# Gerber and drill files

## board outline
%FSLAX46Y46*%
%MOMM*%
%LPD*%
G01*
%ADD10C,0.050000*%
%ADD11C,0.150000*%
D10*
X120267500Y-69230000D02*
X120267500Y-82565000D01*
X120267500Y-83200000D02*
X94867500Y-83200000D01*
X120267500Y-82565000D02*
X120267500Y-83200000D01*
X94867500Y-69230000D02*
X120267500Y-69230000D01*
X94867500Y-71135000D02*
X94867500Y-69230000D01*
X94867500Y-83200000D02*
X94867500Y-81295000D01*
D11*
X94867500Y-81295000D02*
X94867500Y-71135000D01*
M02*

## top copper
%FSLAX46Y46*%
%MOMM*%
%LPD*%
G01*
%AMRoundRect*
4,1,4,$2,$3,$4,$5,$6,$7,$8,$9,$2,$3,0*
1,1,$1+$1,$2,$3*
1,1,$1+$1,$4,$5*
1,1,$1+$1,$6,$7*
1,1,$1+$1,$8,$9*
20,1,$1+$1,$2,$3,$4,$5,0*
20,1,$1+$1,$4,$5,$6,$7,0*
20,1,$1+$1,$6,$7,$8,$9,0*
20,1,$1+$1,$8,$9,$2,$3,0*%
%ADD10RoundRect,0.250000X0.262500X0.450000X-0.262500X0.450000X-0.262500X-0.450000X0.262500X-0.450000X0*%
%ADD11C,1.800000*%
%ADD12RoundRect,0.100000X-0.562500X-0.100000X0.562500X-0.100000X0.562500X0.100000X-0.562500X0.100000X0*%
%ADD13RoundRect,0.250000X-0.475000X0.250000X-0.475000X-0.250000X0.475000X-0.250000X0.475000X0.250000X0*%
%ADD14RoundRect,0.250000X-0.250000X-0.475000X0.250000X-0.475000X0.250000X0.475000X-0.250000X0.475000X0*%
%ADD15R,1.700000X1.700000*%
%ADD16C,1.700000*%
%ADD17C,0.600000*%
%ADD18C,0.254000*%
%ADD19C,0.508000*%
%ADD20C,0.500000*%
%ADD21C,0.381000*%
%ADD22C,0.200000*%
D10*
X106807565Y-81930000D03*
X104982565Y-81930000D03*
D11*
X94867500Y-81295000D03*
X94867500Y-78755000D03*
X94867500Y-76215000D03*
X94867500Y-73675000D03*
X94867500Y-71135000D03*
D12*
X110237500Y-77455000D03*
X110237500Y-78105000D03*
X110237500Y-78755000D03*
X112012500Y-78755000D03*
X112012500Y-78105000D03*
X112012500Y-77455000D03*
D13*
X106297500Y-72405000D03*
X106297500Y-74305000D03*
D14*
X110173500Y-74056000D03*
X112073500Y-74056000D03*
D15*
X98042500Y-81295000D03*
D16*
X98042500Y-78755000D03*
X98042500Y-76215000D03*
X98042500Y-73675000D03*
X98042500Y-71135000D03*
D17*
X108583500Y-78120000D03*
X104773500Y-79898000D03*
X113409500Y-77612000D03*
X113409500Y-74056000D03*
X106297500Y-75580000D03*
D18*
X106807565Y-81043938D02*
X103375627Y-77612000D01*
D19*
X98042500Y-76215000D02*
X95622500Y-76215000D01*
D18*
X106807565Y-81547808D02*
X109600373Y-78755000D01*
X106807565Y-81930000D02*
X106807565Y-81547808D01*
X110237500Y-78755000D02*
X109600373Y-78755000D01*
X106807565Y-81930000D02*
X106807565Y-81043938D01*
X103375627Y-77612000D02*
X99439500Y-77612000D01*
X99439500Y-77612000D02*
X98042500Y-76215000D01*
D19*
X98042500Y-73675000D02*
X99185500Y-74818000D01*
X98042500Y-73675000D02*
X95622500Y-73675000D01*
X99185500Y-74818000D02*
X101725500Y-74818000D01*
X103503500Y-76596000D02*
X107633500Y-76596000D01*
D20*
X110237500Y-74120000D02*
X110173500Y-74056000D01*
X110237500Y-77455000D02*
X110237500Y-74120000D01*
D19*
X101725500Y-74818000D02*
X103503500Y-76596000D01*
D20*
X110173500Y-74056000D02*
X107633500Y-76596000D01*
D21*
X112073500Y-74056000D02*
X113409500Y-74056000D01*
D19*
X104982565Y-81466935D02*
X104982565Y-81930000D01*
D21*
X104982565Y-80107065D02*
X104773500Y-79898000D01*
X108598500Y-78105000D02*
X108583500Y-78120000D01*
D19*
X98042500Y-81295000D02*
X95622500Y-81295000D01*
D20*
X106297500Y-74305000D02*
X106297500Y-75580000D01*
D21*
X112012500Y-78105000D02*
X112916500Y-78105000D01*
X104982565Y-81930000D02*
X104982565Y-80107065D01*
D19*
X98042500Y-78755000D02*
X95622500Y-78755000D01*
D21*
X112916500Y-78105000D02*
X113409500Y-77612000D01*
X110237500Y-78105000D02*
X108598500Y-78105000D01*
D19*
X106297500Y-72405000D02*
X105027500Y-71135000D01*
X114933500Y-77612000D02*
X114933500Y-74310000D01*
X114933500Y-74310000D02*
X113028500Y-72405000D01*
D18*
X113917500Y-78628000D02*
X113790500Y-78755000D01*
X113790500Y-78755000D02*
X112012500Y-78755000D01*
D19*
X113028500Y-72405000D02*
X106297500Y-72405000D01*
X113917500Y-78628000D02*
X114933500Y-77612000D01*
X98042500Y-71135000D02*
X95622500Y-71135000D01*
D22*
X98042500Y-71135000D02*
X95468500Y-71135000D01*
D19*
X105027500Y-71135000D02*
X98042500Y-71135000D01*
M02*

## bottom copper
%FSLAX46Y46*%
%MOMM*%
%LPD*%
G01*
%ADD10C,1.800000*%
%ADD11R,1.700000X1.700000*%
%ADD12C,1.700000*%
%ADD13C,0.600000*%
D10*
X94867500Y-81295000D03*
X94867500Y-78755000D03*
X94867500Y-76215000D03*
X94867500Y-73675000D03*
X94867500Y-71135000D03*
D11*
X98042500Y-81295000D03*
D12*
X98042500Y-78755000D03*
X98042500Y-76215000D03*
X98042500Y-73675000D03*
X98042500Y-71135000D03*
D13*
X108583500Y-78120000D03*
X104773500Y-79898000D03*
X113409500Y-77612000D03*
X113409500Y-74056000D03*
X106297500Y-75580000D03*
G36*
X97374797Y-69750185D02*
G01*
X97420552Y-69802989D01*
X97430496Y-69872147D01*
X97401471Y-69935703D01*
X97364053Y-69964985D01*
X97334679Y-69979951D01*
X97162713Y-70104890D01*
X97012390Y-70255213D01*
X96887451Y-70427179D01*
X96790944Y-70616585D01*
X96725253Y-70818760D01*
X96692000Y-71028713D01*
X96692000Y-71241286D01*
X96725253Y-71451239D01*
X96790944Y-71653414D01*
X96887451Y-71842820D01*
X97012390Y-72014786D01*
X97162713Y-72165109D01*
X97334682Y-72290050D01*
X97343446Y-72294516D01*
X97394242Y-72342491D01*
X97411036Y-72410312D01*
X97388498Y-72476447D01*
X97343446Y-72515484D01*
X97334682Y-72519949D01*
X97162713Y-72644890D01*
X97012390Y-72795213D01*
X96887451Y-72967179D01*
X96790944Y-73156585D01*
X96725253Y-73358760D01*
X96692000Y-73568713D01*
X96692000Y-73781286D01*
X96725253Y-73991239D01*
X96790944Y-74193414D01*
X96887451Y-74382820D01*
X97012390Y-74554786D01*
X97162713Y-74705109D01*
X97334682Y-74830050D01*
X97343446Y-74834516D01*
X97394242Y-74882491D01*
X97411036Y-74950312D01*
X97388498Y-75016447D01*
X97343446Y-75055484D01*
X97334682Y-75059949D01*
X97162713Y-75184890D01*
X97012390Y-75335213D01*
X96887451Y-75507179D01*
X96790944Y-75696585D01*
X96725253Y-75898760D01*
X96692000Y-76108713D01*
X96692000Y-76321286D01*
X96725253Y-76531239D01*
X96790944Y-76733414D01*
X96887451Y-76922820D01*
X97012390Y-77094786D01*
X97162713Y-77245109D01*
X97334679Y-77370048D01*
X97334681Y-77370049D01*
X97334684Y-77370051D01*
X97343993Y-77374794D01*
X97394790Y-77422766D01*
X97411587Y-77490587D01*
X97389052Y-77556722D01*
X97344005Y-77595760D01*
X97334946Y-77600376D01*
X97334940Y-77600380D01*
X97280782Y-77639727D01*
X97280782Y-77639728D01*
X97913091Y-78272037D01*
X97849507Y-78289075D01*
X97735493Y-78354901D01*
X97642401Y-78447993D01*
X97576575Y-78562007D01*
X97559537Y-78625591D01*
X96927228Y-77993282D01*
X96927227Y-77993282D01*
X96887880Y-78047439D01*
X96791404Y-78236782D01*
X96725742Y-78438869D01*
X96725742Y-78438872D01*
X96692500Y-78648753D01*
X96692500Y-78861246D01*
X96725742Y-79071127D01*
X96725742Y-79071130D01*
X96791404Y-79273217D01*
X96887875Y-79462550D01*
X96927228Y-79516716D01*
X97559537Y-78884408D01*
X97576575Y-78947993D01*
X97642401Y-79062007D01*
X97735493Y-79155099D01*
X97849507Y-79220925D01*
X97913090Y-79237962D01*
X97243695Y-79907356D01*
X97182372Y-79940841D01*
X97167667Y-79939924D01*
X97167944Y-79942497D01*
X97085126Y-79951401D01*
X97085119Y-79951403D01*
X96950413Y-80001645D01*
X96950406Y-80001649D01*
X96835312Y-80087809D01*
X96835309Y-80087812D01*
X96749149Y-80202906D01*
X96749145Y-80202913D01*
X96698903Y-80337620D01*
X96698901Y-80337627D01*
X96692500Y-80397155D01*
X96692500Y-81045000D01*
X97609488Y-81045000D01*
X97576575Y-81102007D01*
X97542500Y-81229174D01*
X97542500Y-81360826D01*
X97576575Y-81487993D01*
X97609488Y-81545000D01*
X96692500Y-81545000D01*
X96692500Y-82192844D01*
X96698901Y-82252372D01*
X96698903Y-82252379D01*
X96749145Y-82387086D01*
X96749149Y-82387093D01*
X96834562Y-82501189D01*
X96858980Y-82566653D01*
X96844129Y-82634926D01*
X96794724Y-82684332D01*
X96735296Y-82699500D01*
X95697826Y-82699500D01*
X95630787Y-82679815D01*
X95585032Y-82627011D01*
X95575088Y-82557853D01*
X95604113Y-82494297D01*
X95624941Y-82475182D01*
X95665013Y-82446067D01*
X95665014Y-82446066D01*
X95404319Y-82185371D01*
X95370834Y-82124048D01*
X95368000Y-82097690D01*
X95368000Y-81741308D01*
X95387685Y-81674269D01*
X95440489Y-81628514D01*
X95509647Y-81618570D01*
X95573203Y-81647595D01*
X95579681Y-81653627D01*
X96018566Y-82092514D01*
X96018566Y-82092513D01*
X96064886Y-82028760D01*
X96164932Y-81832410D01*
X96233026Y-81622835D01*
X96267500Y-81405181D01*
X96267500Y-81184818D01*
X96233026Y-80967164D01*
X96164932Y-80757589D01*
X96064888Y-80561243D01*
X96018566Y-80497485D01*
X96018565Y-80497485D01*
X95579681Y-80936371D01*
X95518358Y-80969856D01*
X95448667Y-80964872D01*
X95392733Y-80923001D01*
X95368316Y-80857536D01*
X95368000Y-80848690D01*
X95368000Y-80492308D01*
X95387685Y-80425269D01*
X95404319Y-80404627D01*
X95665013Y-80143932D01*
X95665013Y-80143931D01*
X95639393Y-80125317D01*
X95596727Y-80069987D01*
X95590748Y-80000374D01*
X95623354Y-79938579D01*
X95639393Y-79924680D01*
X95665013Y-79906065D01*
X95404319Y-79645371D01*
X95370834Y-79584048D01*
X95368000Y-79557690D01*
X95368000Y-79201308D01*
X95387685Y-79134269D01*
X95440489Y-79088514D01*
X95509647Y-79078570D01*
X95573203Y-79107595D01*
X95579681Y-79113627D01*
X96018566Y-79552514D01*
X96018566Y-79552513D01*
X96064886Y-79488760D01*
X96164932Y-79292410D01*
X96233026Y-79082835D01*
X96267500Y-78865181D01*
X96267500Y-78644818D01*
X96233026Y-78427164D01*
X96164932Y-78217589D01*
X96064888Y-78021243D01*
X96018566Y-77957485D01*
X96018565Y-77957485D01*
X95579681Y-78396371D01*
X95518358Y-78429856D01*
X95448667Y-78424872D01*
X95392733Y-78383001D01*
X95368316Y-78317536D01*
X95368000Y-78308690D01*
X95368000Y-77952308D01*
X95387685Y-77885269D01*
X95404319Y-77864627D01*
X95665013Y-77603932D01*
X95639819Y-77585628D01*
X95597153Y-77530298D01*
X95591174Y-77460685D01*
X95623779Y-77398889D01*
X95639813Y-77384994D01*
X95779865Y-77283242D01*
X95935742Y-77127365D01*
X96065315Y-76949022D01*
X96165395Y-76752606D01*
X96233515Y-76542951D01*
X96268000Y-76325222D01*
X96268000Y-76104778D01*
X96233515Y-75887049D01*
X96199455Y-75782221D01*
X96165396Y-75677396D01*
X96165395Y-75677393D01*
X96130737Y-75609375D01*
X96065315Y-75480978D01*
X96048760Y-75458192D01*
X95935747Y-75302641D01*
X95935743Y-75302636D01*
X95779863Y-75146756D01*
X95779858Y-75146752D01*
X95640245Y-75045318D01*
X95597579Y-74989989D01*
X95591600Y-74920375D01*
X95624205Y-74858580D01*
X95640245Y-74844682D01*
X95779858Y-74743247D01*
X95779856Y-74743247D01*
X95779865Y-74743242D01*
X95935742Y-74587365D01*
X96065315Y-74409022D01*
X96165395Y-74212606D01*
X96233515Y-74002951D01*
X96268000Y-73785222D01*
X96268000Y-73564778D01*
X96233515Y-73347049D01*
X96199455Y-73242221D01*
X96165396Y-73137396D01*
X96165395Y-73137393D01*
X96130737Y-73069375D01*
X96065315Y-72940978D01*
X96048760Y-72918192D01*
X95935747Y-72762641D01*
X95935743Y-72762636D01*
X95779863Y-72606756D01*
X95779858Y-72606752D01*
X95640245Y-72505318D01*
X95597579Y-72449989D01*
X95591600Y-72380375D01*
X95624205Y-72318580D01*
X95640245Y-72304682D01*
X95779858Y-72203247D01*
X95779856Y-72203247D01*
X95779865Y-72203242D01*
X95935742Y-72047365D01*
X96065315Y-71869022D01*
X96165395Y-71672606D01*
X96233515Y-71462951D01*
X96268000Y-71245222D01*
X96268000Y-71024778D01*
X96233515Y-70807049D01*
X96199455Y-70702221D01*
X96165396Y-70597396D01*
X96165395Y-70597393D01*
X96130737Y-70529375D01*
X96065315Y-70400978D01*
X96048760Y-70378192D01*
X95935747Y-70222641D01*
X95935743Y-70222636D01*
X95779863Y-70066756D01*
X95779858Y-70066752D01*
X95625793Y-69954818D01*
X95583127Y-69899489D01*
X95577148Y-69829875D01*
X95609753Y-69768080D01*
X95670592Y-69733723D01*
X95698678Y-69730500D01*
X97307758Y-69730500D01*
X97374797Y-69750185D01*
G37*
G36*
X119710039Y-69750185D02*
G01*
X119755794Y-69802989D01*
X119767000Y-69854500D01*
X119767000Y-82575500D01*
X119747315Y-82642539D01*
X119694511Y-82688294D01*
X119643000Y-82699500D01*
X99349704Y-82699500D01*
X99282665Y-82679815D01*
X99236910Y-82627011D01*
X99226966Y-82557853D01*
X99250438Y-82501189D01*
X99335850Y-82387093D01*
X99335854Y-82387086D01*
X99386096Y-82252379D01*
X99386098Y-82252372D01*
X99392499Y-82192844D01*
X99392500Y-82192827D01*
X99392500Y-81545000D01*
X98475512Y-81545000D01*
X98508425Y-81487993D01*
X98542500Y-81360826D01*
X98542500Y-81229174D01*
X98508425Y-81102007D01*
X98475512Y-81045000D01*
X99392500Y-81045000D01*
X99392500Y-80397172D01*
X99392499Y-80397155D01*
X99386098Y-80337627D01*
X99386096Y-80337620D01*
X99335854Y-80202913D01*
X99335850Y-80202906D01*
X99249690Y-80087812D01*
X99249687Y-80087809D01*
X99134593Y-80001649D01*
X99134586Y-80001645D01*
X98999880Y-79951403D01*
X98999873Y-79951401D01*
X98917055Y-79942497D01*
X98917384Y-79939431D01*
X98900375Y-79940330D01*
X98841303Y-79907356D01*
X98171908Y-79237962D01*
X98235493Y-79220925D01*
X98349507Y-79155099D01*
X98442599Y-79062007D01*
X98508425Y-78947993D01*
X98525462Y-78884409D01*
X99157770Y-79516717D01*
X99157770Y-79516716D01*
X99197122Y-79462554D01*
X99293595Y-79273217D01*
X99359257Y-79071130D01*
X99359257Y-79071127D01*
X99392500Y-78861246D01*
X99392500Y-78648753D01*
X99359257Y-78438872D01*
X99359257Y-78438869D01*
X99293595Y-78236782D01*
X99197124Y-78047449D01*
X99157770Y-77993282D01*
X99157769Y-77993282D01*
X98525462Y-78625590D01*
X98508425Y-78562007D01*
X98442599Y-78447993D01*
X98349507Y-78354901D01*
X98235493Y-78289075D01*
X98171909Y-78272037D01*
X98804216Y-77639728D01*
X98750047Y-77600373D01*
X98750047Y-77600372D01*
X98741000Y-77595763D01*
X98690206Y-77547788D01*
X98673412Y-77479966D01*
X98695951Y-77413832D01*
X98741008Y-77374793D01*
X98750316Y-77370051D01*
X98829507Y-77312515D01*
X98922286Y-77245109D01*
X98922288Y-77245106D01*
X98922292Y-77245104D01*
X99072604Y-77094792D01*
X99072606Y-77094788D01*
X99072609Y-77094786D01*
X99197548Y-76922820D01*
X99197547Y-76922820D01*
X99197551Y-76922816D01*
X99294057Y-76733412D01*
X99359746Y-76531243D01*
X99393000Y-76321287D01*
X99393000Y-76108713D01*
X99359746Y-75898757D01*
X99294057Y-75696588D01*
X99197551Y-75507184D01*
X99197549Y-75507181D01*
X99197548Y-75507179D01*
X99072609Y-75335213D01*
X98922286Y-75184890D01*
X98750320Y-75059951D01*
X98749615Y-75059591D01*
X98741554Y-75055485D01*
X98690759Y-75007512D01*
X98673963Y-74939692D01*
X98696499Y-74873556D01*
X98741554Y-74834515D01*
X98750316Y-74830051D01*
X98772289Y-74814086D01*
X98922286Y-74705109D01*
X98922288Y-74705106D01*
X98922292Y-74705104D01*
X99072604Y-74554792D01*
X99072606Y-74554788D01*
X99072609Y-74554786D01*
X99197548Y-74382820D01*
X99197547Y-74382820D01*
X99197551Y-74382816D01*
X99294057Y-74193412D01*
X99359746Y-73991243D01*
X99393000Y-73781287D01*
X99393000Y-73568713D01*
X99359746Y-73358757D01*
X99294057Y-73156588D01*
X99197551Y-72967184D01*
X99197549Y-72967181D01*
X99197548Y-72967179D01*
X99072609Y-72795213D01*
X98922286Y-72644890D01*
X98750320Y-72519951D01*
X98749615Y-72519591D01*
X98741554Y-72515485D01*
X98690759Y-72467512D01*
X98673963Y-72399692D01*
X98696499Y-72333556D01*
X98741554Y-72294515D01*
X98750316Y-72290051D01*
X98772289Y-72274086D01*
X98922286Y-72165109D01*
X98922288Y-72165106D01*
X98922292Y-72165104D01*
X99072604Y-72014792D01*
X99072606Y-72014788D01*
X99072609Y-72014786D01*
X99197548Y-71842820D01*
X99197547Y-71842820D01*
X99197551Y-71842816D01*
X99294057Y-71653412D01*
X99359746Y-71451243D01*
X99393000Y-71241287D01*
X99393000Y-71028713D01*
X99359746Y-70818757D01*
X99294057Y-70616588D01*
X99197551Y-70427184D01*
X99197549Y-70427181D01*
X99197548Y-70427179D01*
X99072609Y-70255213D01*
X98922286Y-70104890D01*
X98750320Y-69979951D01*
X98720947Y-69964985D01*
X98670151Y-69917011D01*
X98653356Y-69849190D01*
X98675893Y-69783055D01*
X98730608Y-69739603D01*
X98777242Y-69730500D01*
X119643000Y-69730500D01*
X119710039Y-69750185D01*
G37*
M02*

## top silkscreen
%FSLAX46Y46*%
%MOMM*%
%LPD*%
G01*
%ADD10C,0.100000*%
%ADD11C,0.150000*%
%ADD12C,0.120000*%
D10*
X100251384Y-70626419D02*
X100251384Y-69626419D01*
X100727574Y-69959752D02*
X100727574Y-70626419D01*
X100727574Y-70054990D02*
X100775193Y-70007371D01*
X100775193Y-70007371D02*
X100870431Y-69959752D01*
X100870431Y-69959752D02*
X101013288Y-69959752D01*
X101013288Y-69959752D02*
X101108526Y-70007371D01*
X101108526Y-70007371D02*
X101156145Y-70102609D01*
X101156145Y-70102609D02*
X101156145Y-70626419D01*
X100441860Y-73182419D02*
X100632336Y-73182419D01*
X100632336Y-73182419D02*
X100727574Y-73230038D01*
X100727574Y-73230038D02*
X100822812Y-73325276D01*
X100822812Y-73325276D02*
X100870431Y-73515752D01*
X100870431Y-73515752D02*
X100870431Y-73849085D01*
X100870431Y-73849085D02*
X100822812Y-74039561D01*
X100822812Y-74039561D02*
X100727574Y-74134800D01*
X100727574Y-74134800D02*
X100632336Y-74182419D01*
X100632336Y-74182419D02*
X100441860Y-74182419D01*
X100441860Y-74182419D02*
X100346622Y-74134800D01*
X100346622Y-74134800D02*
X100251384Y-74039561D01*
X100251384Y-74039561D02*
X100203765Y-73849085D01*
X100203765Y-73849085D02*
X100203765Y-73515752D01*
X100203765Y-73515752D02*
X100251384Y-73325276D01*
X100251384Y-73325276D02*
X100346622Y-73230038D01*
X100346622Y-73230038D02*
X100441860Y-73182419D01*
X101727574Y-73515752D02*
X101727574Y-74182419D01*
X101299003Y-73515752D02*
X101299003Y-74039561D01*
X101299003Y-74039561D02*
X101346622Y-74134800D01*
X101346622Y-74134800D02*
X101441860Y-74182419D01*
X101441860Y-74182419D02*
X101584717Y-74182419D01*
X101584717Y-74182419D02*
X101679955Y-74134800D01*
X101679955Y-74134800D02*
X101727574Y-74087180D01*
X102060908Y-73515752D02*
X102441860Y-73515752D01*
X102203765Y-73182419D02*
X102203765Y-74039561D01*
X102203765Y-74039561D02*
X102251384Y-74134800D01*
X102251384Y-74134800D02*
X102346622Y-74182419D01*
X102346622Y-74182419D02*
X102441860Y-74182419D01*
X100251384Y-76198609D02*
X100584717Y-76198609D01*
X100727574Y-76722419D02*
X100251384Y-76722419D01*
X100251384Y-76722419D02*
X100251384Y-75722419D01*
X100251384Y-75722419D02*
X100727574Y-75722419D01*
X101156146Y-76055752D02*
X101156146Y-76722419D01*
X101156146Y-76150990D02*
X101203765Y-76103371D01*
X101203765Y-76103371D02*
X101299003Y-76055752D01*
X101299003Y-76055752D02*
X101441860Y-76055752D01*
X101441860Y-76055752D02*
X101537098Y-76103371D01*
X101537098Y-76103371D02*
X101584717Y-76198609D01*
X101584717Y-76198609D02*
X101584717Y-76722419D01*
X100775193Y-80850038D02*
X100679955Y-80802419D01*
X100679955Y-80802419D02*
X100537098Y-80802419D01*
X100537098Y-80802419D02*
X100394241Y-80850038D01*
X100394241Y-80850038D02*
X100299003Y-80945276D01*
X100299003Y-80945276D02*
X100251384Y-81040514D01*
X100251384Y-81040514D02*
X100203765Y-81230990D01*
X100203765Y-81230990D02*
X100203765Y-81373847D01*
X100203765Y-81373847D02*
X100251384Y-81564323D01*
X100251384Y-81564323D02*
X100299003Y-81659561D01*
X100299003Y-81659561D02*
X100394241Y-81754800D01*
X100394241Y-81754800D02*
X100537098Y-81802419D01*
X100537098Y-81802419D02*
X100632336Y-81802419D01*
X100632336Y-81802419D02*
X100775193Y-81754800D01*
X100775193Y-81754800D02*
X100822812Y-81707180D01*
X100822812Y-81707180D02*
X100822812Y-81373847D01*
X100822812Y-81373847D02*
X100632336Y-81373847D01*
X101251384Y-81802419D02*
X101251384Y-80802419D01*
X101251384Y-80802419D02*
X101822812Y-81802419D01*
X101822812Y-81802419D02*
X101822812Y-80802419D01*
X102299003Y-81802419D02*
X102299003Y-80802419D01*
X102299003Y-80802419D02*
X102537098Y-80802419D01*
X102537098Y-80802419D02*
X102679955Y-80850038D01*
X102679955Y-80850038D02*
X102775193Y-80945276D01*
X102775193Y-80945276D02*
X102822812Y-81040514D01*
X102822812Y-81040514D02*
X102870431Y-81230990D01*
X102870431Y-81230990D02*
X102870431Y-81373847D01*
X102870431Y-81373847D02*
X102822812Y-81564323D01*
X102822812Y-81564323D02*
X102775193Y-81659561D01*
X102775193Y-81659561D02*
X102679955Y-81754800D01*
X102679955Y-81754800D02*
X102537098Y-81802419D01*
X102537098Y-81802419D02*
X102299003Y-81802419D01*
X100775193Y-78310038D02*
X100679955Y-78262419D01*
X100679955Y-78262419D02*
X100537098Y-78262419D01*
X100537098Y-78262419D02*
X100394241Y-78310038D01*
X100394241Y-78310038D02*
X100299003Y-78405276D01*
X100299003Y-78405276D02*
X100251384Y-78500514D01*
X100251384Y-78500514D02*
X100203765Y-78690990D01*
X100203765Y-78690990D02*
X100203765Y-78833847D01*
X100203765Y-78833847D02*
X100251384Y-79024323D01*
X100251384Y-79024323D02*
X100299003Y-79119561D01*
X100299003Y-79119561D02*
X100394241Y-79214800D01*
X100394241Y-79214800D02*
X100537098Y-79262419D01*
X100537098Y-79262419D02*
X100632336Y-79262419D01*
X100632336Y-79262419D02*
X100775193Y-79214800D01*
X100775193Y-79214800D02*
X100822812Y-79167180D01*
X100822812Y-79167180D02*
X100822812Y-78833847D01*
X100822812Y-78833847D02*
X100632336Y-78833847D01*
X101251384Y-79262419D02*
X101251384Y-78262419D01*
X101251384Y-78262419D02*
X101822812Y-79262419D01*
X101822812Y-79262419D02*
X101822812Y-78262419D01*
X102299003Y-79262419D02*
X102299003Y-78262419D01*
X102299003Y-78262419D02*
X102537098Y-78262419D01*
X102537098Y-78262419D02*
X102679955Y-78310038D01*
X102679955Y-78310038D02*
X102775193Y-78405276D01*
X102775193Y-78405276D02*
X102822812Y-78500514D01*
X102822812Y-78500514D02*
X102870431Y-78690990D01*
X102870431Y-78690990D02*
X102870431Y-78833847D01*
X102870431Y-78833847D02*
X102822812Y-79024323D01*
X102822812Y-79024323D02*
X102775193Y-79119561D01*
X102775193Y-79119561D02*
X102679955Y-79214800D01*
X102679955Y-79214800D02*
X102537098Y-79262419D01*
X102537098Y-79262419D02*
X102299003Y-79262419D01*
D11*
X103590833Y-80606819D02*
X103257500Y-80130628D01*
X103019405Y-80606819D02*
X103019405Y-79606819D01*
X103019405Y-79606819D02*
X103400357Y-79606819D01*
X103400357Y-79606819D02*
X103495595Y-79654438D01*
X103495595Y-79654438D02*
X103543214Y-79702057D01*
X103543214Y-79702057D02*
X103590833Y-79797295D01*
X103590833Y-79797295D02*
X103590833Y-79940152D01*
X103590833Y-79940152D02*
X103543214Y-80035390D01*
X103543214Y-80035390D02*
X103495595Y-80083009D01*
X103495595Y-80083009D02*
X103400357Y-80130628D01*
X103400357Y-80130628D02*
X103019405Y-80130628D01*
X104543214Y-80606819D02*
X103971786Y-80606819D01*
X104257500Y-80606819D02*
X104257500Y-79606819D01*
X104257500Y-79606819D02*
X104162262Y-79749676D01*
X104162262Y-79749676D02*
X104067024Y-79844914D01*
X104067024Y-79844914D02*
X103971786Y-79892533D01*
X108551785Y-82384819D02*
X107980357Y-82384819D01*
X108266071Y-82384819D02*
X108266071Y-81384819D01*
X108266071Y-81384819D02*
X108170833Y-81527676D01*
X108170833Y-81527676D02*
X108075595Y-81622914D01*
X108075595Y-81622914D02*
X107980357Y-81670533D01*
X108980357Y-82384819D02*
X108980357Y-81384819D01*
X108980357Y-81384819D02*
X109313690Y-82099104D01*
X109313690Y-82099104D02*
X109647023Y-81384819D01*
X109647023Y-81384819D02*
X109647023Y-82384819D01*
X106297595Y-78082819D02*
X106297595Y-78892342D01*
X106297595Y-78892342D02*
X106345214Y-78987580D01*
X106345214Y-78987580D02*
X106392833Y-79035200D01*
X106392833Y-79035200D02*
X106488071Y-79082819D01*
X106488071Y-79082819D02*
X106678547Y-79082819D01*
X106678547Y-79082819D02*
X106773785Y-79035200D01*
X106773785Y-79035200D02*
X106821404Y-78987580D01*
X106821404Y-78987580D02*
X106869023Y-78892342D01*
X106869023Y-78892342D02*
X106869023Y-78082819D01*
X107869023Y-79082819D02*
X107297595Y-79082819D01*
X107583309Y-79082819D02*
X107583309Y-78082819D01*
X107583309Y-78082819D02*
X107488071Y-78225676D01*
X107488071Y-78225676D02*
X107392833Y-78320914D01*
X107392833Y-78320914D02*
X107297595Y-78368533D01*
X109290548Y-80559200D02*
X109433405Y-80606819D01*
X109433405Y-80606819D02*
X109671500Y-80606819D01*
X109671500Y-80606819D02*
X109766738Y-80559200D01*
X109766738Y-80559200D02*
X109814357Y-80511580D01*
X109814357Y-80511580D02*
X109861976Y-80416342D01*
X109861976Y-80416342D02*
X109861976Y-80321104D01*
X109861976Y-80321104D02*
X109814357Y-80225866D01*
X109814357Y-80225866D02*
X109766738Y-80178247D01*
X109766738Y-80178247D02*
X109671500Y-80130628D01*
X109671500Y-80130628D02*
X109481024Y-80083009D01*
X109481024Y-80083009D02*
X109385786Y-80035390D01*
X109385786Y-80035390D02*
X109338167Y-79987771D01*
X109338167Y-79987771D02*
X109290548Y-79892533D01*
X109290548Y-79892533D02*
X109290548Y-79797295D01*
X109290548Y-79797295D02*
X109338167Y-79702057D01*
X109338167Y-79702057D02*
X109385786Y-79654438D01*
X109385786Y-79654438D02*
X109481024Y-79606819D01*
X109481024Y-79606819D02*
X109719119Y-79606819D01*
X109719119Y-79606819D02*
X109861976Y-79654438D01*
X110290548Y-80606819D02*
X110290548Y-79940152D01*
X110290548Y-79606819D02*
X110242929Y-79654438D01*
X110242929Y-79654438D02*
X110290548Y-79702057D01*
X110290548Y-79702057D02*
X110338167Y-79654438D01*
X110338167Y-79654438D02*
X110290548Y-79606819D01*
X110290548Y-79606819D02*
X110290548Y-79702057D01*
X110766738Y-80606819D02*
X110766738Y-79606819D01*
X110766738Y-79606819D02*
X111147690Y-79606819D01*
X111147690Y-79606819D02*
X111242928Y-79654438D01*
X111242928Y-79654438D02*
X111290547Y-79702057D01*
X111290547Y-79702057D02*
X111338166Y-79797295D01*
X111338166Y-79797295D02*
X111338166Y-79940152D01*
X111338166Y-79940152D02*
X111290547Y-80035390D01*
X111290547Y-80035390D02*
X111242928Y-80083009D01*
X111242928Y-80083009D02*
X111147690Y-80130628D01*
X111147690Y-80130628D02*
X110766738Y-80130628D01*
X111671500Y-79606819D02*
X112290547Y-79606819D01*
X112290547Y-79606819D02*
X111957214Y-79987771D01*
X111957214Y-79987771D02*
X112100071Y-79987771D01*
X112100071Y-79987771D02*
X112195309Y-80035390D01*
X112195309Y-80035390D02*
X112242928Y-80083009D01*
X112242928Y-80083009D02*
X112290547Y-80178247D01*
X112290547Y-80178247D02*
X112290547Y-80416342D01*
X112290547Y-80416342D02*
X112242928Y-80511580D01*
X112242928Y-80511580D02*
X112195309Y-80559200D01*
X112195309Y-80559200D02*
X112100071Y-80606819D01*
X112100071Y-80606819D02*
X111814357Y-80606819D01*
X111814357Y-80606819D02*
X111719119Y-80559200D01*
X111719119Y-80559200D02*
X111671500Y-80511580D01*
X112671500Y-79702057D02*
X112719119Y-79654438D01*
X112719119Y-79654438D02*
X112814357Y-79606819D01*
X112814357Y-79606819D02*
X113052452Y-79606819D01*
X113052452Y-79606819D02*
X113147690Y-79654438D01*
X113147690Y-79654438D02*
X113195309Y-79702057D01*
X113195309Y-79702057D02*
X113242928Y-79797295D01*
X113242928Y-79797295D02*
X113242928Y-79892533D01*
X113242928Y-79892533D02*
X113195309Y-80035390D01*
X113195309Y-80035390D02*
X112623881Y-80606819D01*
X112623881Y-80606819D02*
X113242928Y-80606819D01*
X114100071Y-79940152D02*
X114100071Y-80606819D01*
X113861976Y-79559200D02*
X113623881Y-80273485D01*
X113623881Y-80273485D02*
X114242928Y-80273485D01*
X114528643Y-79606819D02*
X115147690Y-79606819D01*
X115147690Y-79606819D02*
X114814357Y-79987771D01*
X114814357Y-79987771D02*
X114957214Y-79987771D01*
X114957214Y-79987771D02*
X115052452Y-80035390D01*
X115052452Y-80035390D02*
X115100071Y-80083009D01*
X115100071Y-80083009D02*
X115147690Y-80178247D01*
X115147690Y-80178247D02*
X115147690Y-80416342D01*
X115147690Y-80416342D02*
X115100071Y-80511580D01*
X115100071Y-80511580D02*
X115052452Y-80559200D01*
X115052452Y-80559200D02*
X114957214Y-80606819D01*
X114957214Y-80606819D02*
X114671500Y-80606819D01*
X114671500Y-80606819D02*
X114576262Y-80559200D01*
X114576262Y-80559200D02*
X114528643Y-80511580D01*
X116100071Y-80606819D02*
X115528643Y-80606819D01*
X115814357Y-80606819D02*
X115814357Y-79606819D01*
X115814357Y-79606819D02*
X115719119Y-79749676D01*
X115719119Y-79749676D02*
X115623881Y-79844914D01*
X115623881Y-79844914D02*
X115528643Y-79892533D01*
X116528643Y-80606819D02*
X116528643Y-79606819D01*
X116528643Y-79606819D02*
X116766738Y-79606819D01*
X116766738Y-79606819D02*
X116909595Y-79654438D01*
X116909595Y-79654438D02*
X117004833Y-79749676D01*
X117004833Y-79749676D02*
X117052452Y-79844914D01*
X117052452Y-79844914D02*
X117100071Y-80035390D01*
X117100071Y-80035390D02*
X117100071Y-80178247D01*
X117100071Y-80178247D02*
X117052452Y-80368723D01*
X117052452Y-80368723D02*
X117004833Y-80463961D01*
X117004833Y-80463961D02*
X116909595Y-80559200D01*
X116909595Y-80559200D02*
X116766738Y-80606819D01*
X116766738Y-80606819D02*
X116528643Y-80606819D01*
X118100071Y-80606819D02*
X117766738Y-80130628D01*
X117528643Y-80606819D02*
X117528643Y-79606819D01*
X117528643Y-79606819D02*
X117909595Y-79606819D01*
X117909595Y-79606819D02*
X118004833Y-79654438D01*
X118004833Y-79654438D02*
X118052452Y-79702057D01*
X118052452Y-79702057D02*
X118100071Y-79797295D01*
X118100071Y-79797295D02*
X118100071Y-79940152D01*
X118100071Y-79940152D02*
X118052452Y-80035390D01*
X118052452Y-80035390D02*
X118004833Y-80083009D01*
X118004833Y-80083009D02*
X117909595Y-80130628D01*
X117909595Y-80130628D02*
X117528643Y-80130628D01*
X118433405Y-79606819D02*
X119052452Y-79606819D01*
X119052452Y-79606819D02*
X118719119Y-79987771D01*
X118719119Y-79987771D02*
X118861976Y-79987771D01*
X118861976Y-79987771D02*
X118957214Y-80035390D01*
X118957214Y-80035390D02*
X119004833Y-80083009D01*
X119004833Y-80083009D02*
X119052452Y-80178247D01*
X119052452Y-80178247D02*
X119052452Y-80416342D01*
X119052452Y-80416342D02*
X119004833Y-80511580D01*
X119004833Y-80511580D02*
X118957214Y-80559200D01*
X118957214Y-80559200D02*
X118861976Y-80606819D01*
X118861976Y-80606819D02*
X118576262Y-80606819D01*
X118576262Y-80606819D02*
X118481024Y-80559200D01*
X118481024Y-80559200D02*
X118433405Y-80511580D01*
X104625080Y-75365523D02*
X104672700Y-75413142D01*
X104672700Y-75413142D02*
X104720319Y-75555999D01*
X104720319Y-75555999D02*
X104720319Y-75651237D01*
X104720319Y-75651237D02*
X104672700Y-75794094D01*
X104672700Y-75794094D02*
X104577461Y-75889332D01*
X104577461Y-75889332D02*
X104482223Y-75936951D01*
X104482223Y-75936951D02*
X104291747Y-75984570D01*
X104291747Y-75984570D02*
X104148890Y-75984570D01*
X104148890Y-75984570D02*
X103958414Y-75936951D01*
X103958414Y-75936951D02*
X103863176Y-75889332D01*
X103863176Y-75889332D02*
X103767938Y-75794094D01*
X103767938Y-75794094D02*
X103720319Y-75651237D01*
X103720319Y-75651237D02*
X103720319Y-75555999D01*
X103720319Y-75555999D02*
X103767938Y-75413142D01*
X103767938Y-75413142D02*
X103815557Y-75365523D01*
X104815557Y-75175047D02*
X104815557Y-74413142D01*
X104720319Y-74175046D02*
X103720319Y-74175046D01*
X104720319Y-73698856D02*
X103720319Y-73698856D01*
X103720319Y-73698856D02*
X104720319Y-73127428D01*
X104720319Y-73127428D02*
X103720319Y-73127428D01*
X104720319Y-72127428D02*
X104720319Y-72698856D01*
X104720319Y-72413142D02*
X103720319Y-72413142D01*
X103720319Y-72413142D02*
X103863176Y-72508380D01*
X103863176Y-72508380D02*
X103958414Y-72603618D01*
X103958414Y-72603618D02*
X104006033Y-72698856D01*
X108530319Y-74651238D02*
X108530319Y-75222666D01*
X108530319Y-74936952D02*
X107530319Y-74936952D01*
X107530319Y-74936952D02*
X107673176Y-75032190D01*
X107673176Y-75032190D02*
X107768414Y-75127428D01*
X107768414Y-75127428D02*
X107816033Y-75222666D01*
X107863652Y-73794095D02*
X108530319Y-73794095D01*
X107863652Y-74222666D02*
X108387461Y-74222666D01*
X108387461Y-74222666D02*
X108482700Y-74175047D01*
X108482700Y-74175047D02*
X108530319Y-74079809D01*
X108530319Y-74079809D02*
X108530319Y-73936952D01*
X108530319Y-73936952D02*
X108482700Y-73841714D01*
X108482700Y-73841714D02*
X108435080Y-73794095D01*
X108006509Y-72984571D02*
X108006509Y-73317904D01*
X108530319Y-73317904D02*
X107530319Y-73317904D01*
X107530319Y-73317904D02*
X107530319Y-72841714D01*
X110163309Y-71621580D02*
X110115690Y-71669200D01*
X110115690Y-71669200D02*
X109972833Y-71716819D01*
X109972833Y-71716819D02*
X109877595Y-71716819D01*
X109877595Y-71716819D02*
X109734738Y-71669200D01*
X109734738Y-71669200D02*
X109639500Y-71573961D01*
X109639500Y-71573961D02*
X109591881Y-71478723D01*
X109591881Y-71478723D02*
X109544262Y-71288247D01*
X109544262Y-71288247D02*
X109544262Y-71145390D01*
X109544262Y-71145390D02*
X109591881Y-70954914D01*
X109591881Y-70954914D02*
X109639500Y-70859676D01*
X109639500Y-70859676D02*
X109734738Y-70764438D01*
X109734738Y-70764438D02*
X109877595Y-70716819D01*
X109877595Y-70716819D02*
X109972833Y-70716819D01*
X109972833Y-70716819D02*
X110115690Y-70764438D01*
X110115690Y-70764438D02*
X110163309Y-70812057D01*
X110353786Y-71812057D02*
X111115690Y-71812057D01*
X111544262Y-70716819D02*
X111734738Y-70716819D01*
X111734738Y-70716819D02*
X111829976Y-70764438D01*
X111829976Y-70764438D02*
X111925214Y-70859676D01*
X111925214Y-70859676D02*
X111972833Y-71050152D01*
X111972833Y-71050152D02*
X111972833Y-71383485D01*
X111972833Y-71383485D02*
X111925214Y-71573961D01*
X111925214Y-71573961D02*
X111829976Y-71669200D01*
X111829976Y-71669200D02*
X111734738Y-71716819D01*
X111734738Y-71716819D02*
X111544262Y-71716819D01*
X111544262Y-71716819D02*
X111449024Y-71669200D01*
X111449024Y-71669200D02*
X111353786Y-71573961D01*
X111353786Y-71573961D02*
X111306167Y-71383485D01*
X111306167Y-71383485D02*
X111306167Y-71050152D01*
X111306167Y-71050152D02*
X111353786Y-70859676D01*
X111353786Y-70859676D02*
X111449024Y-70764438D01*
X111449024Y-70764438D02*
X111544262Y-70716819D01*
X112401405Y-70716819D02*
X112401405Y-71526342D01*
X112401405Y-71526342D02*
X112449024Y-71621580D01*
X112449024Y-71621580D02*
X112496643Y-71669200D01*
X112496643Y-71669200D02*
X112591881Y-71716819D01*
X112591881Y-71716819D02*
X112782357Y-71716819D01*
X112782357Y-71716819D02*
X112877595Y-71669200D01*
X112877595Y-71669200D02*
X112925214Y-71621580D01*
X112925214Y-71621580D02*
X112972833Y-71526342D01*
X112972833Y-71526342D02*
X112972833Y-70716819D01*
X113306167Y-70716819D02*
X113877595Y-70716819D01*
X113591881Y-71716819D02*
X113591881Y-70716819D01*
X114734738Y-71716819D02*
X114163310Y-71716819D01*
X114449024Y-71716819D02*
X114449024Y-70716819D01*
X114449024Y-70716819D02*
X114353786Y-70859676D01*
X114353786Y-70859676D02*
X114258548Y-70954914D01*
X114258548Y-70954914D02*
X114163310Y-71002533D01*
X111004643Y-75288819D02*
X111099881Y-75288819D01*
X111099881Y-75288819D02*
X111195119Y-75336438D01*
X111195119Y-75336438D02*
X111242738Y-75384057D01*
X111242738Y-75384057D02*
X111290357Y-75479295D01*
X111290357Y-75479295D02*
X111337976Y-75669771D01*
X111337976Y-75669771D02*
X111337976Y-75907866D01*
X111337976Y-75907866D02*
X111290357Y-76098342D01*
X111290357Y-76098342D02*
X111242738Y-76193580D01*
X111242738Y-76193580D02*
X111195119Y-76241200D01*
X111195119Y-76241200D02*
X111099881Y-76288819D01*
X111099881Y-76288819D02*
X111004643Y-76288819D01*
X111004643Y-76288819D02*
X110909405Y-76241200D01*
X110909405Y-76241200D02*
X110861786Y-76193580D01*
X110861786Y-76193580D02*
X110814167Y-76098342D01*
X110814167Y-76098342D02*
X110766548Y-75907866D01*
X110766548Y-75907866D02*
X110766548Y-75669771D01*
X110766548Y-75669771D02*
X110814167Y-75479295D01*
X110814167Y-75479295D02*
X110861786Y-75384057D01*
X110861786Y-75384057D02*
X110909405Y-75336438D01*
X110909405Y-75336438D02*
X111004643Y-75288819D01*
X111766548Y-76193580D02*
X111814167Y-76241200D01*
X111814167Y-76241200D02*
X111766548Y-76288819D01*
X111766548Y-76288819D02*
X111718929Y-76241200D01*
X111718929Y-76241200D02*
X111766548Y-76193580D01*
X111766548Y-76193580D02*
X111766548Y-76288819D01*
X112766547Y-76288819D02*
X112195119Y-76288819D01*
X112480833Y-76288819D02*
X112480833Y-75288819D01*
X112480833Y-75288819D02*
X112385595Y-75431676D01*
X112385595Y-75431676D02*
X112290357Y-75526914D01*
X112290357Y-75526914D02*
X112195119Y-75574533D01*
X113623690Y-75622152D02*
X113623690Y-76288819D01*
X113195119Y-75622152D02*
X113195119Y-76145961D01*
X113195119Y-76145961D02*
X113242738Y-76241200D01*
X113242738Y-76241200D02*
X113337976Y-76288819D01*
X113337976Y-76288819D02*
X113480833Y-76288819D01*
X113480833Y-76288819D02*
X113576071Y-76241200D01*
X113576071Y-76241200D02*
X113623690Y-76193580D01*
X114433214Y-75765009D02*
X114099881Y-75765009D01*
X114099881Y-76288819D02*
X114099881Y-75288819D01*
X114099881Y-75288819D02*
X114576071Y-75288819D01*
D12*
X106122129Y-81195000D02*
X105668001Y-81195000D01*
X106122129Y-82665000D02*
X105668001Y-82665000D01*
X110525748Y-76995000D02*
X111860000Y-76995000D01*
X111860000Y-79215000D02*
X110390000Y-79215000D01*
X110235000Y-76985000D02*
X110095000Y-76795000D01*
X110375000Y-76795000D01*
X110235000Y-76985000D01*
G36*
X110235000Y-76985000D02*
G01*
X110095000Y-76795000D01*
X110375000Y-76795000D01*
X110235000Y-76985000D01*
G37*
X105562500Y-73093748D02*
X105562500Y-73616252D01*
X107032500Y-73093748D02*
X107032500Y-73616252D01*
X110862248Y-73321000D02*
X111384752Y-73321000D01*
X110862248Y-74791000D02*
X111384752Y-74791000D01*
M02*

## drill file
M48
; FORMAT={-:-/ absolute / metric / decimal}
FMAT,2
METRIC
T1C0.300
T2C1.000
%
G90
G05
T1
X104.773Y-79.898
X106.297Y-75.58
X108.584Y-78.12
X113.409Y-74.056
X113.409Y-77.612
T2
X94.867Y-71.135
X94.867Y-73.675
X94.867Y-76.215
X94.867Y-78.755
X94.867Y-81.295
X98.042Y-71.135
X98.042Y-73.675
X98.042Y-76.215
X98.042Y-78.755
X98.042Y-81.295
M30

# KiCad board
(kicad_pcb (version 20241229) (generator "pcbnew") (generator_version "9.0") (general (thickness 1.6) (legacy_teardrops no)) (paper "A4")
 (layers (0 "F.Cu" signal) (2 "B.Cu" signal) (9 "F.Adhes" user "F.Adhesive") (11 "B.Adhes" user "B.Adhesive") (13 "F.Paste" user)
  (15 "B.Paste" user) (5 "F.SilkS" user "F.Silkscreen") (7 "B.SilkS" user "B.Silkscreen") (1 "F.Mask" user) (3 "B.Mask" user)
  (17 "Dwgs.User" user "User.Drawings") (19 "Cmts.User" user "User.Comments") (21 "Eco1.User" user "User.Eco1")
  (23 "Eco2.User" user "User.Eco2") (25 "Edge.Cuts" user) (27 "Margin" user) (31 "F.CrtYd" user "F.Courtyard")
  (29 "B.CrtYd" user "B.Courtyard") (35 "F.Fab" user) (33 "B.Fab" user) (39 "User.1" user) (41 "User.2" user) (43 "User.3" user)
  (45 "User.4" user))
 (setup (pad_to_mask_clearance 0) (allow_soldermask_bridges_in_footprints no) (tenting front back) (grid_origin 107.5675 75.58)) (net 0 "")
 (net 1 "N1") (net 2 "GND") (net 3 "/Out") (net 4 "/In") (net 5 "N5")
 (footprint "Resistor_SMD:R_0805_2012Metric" (layer "F.Cu") (at 105.895065 81.93 180)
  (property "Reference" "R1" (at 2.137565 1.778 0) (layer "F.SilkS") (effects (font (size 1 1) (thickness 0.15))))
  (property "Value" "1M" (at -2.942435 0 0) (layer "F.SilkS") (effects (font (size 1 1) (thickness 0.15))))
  (fp_line (start -0.227064 0.735) (end 0.227064 0.735) (stroke (width 0.12) (type solid)) (layer "F.SilkS"))
  (fp_line (start -0.227064 -0.735) (end 0.227064 -0.735) (stroke (width 0.12) (type solid)) (layer "F.SilkS"))
  (pad "1" smd roundrect (at -0.9125 0 180) (size 1.025 1.4) (layers "F.Cu" "F.Mask" "F.Paste") (roundrect_rratio 0.243902) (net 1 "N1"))
  (pad "2" smd roundrect (at 0.9125 0 180) (size 1.025 1.4) (layers "F.Cu" "F.Mask" "F.Paste") (roundrect_rratio 0.243902) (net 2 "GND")))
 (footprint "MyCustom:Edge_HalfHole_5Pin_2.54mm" (layer "F.Cu") (at 94.8675 81.295 90)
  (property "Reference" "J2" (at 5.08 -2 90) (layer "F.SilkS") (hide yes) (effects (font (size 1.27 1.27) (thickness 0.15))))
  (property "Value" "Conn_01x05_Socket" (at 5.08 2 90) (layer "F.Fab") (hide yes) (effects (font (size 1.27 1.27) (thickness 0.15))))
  (fp_line (start 0 0) (end 10.16 0) (stroke (width 0.15) (type solid)) (layer "Edge.Cuts"))
  (pad "1" thru_hole circle (at 0 0 90) (size 1.8 1.8) (drill 1) (layers "*.Cu" "*.Mask") (remove_unused_layers no) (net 2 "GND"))
  (pad "2" thru_hole circle (at 2.54 0 90) (size 1.8 1.8) (drill 1) (layers "*.Cu" "*.Mask") (remove_unused_layers no) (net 2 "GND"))
  (pad "3" thru_hole circle (at 5.08 0 90) (size 1.8 1.8) (drill 1) (layers "*.Cu" "*.Mask") (remove_unused_layers no) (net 1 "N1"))
  (pad "4" thru_hole circle (at 7.62 0 90) (size 1.8 1.8) (drill 1) (layers "*.Cu" "*.Mask") (remove_unused_layers no) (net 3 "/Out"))
  (pad "5" thru_hole circle (at 10.16 0 90) (size 1.8 1.8) (drill 1) (layers "*.Cu" "*.Mask") (remove_unused_layers no) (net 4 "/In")))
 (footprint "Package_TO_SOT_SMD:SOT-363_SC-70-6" (layer "F.Cu") (at 111.125 78.105)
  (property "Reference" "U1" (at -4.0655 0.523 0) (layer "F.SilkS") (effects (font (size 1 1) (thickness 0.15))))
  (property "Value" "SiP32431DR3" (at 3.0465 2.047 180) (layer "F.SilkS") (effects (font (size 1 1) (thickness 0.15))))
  (fp_line (start -0.599252 -1.11) (end 0.735 -1.11) (stroke (width 0.12) (type solid)) (layer "F.SilkS"))
  (fp_line (start 0.735 1.11) (end -0.735 1.11) (stroke (width 0.12) (type solid)) (layer "F.SilkS"))
  (fp_poly (pts (xy -0.89 -1.12) (xy -1.03 -1.31) (xy -0.75 -1.31)) (stroke (width 0.12) (type solid)) (fill yes) (layer "F.SilkS"))
  (pad "1" smd roundrect (at -0.8875 -0.65) (size 1.325 0.4) (layers "F.Cu" "F.Mask" "F.Paste") (roundrect_rratio 0.25) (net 3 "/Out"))
  (pad "2" smd roundrect (at -0.8875 0) (size 1.325 0.4) (layers "F.Cu" "F.Mask" "F.Paste") (roundrect_rratio 0.25) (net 2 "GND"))
  (pad "3" smd roundrect (at -0.8875 0.65) (size 1.325 0.4) (layers "F.Cu" "F.Mask" "F.Paste") (roundrect_rratio 0.25) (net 1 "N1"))
  (pad "4" smd roundrect (at 0.8875 0.65) (size 1.325 0.4) (layers "F.Cu" "F.Mask" "F.Paste") (roundrect_rratio 0.25) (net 4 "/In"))
  (pad "5" smd roundrect (at 0.8875 0) (size 1.325 0.4) (layers "F.Cu" "F.Mask" "F.Paste") (roundrect_rratio 0.25) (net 2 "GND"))
  (pad "6" smd roundrect (at 0.8875 -0.65) (size 1.325 0.4) (layers "F.Cu" "F.Mask" "F.Paste") (roundrect_rratio 0.25) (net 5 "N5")))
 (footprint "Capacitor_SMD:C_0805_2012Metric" (layer "F.Cu") (at 106.2975 73.355 -90)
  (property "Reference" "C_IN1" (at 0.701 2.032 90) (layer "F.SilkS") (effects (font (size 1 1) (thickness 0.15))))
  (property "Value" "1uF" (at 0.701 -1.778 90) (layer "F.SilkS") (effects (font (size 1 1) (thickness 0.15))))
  (fp_line (start -0.261252 0.735) (end 0.261252 0.735) (stroke (width 0.12) (type solid)) (layer "F.SilkS"))
  (fp_line (start -0.261252 -0.735) (end 0.261252 -0.735) (stroke (width 0.12) (type solid)) (layer "F.SilkS"))
  (pad "1" smd roundrect (at -0.95 0 270) (size 1 1.45) (layers "F.Cu" "F.Mask" "F.Paste") (roundrect_rratio 0.25) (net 4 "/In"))
  (pad "2" smd roundrect (at 0.95 0 270) (size 1 1.45) (layers "F.Cu" "F.Mask" "F.Paste") (roundrect_rratio 0.25) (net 2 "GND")))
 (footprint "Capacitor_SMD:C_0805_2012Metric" (layer "F.Cu") (at 111.1235 74.056)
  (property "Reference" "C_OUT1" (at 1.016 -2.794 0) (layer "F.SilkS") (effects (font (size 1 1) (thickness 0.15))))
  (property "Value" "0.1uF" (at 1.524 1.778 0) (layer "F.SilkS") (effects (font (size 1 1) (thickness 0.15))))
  (fp_line (start -0.261252 -0.735) (end 0.261252 -0.735) (stroke (width 0.12) (type solid)) (layer "F.SilkS"))
  (fp_line (start -0.261252 0.735) (end 0.261252 0.735) (stroke (width 0.12) (type solid)) (layer "F.SilkS"))
  (pad "1" smd roundrect (at -0.95 0) (size 1 1.45) (layers "F.Cu" "F.Mask" "F.Paste") (roundrect_rratio 0.25) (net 3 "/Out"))
  (pad "2" smd roundrect (at 0.95 0) (size 1 1.45) (layers "F.Cu" "F.Mask" "F.Paste") (roundrect_rratio 0.25) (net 2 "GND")))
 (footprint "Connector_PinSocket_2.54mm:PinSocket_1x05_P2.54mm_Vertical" (layer "B.Cu") (at 98.0425 81.295)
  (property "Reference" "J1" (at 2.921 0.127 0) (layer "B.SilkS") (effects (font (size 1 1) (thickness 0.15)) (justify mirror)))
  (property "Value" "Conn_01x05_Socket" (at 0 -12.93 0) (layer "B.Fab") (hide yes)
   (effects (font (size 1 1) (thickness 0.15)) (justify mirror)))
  (pad "1" thru_hole rect (at 0 0) (size 1.7 1.7) (drill 1) (layers "*.Cu" "*.Mask") (remove_unused_layers no) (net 2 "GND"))
  (pad "2" thru_hole circle (at 0 -2.54) (size 1.7 1.7) (drill 1) (layers "*.Cu" "*.Mask") (remove_unused_layers no) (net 2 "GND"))
  (pad "3" thru_hole circle (at 0 -5.08) (size 1.7 1.7) (drill 1) (layers "*.Cu" "*.Mask") (remove_unused_layers no) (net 1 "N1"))
  (pad "4" thru_hole circle (at 0 -7.62) (size 1.7 1.7) (drill 1) (layers "*.Cu" "*.Mask") (remove_unused_layers no) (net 3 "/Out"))
  (pad "5" thru_hole circle (at 0 -10.16) (size 1.7 1.7) (drill 1) (layers "*.Cu" "*.Mask") (remove_unused_layers no) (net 4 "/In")))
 (gr_line (start 120.2675 69.23) (end 120.2675 82.565) (stroke (width 0.05) (type default)) (layer "Edge.Cuts"))
 (gr_line (start 120.2675 83.2) (end 94.8675 83.2) (stroke (width 0.05) (type default)) (layer "Edge.Cuts"))
 (gr_line (start 120.2675 82.565) (end 120.2675 83.2) (stroke (width 0.05) (type default)) (layer "Edge.Cuts"))
 (gr_line (start 94.8675 69.23) (end 120.2675 69.23) (stroke (width 0.05) (type default)) (layer "Edge.Cuts"))
 (gr_line (start 94.8675 71.135) (end 94.8675 69.23) (stroke (width 0.05) (type default)) (layer "Edge.Cuts"))
 (gr_line (start 94.8675 83.2) (end 94.8675 81.295) (stroke (width 0.05) (type default)) (layer "Edge.Cuts"))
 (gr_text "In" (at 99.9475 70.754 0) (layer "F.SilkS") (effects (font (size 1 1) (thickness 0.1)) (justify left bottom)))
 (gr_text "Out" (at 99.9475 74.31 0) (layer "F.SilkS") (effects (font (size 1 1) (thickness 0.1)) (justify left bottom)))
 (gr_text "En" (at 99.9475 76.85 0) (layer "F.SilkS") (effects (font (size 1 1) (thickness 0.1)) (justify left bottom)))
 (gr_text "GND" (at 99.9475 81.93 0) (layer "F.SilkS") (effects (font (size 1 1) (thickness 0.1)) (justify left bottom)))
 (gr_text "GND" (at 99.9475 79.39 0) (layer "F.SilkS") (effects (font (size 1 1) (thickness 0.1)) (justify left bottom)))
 (segment (start 106.807565 81.043938) (end 103.375627 77.612) (width 0.254) (layer "F.Cu") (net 1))
 (segment (start 98.0425 76.215) (end 95.6225 76.215) (width 0.508) (layer "F.Cu") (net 1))
 (segment (start 106.807565 81.547808) (end 109.600373 78.755) (width 0.254) (layer "F.Cu") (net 1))
 (segment (start 106.807565 81.93) (end 106.807565 81.547808) (width 0.254) (layer "F.Cu") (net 1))
 (segment (start 110.2375 78.755) (end 109.600373 78.755) (width 0.254) (layer "F.Cu") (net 1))
 (segment (start 106.807565 81.93) (end 106.807565 81.043938) (width 0.254) (layer "F.Cu") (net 1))
 (segment (start 103.375627 77.612) (end 99.4395 77.612) (width 0.254) (layer "F.Cu") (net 1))
 (segment (start 99.4395 77.612) (end 98.0425 76.215) (width 0.254) (layer "F.Cu") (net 1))
 (segment (start 98.0425 73.675) (end 99.1855 74.818) (width 0.508) (layer "F.Cu") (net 3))
 (segment (start 98.0425 73.675) (end 95.6225 73.675) (width 0.508) (layer "F.Cu") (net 3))
 (segment (start 99.1855 74.818) (end 101.7255 74.818) (width 0.508) (layer "F.Cu") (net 3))
 (segment (start 103.5035 76.596) (end 107.6335 76.596) (width 0.508) (layer "F.Cu") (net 3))
 (segment (start 110.2375 74.12) (end 110.1735 74.056) (width 0.5) (layer "F.Cu") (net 3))
 (segment (start 110.2375 77.455) (end 110.2375 74.12) (width 0.5) (layer "F.Cu") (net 3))
 (segment (start 101.7255 74.818) (end 103.5035 76.596) (width 0.508) (layer "F.Cu") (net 3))
 (segment (start 110.1735 74.056) (end 107.6335 76.596) (width 0.5) (layer "F.Cu") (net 3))
 (segment (start 112.0735 74.056) (end 113.4095 74.056) (width 0.381) (layer "F.Cu") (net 2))
 (segment (start 104.982565 81.466935) (end 104.982565 81.93) (width 0.508) (layer "F.Cu") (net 2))
 (segment (start 104.982565 80.107065) (end 104.7735 79.898) (width 0.381) (layer "F.Cu") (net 2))
 (segment (start 108.5985 78.105) (end 108.5835 78.12) (width 0.381) (layer "F.Cu") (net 2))
 (segment (start 98.0425 81.295) (end 95.6225 81.295) (width 0.508) (layer "F.Cu") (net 2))
 (segment (start 106.2975 74.305) (end 106.2975 75.58) (width 0.5) (layer "F.Cu") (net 2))
 (segment (start 112.0125 78.105) (end 112.9165 78.105) (width 0.381) (layer "F.Cu") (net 2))
 (segment (start 104.982565 81.93) (end 104.982565 80.107065) (width 0.381) (layer "F.Cu") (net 2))
 (segment (start 98.0425 78.755) (end 95.6225 78.755) (width 0.508) (layer "F.Cu") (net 2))
 (segment (start 112.9165 78.105) (end 113.4095 77.612) (width 0.381) (layer "F.Cu") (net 2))
 (segment (start 110.2375 78.105) (end 108.5985 78.105) (width 0.381) (layer "F.Cu") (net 2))
 (via (at 108.5835 78.12) (size 0.6) (drill 0.3) (layers "F.Cu" "B.Cu") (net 2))
 (via (at 104.7735 79.898) (size 0.6) (drill 0.3) (layers "F.Cu" "B.Cu") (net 2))
 (via (at 113.4095 77.612) (size 0.6) (drill 0.3) (layers "F.Cu" "B.Cu") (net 2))
 (via (at 113.4095 74.056) (size 0.6) (drill 0.3) (layers "F.Cu" "B.Cu") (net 2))
 (via (at 106.2975 75.58) (size 0.6) (drill 0.3) (layers "F.Cu" "B.Cu") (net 2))
 (segment (start 106.2975 72.405) (end 105.0275 71.135) (width 0.508) (layer "F.Cu") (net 4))
 (segment (start 114.9335 77.612) (end 114.9335 74.31) (width 0.508) (layer "F.Cu") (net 4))
 (segment (start 114.9335 74.31) (end 113.0285 72.405) (width 0.508) (layer "F.Cu") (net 4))
 (segment (start 113.9175 78.628) (end 113.7905 78.755) (width 0.254) (layer "F.Cu") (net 4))
 (segment (start 113.7905 78.755) (end 112.0125 78.755) (width 0.254) (layer "F.Cu") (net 4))
 (segment (start 113.0285 72.405) (end 106.2975 72.405) (width 0.508) (layer "F.Cu") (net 4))
 (segment (start 113.9175 78.628) (end 114.9335 77.612) (width 0.508) (layer "F.Cu") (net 4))
 (segment (start 98.0425 71.135) (end 95.6225 71.135) (width 0.508) (layer "F.Cu") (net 4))
 (segment (start 98.0425 71.135) (end 95.4685 71.135) (width 0.2) (layer "F.Cu") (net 4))
 (segment (start 105.0275 71.135) (end 98.0425 71.135) (width 0.508) (layer "F.Cu") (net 4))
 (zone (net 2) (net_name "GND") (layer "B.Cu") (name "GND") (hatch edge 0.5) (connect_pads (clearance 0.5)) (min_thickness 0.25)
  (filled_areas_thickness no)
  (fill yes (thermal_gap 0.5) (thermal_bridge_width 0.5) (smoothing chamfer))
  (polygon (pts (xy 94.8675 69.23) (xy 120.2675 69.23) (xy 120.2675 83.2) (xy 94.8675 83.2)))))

